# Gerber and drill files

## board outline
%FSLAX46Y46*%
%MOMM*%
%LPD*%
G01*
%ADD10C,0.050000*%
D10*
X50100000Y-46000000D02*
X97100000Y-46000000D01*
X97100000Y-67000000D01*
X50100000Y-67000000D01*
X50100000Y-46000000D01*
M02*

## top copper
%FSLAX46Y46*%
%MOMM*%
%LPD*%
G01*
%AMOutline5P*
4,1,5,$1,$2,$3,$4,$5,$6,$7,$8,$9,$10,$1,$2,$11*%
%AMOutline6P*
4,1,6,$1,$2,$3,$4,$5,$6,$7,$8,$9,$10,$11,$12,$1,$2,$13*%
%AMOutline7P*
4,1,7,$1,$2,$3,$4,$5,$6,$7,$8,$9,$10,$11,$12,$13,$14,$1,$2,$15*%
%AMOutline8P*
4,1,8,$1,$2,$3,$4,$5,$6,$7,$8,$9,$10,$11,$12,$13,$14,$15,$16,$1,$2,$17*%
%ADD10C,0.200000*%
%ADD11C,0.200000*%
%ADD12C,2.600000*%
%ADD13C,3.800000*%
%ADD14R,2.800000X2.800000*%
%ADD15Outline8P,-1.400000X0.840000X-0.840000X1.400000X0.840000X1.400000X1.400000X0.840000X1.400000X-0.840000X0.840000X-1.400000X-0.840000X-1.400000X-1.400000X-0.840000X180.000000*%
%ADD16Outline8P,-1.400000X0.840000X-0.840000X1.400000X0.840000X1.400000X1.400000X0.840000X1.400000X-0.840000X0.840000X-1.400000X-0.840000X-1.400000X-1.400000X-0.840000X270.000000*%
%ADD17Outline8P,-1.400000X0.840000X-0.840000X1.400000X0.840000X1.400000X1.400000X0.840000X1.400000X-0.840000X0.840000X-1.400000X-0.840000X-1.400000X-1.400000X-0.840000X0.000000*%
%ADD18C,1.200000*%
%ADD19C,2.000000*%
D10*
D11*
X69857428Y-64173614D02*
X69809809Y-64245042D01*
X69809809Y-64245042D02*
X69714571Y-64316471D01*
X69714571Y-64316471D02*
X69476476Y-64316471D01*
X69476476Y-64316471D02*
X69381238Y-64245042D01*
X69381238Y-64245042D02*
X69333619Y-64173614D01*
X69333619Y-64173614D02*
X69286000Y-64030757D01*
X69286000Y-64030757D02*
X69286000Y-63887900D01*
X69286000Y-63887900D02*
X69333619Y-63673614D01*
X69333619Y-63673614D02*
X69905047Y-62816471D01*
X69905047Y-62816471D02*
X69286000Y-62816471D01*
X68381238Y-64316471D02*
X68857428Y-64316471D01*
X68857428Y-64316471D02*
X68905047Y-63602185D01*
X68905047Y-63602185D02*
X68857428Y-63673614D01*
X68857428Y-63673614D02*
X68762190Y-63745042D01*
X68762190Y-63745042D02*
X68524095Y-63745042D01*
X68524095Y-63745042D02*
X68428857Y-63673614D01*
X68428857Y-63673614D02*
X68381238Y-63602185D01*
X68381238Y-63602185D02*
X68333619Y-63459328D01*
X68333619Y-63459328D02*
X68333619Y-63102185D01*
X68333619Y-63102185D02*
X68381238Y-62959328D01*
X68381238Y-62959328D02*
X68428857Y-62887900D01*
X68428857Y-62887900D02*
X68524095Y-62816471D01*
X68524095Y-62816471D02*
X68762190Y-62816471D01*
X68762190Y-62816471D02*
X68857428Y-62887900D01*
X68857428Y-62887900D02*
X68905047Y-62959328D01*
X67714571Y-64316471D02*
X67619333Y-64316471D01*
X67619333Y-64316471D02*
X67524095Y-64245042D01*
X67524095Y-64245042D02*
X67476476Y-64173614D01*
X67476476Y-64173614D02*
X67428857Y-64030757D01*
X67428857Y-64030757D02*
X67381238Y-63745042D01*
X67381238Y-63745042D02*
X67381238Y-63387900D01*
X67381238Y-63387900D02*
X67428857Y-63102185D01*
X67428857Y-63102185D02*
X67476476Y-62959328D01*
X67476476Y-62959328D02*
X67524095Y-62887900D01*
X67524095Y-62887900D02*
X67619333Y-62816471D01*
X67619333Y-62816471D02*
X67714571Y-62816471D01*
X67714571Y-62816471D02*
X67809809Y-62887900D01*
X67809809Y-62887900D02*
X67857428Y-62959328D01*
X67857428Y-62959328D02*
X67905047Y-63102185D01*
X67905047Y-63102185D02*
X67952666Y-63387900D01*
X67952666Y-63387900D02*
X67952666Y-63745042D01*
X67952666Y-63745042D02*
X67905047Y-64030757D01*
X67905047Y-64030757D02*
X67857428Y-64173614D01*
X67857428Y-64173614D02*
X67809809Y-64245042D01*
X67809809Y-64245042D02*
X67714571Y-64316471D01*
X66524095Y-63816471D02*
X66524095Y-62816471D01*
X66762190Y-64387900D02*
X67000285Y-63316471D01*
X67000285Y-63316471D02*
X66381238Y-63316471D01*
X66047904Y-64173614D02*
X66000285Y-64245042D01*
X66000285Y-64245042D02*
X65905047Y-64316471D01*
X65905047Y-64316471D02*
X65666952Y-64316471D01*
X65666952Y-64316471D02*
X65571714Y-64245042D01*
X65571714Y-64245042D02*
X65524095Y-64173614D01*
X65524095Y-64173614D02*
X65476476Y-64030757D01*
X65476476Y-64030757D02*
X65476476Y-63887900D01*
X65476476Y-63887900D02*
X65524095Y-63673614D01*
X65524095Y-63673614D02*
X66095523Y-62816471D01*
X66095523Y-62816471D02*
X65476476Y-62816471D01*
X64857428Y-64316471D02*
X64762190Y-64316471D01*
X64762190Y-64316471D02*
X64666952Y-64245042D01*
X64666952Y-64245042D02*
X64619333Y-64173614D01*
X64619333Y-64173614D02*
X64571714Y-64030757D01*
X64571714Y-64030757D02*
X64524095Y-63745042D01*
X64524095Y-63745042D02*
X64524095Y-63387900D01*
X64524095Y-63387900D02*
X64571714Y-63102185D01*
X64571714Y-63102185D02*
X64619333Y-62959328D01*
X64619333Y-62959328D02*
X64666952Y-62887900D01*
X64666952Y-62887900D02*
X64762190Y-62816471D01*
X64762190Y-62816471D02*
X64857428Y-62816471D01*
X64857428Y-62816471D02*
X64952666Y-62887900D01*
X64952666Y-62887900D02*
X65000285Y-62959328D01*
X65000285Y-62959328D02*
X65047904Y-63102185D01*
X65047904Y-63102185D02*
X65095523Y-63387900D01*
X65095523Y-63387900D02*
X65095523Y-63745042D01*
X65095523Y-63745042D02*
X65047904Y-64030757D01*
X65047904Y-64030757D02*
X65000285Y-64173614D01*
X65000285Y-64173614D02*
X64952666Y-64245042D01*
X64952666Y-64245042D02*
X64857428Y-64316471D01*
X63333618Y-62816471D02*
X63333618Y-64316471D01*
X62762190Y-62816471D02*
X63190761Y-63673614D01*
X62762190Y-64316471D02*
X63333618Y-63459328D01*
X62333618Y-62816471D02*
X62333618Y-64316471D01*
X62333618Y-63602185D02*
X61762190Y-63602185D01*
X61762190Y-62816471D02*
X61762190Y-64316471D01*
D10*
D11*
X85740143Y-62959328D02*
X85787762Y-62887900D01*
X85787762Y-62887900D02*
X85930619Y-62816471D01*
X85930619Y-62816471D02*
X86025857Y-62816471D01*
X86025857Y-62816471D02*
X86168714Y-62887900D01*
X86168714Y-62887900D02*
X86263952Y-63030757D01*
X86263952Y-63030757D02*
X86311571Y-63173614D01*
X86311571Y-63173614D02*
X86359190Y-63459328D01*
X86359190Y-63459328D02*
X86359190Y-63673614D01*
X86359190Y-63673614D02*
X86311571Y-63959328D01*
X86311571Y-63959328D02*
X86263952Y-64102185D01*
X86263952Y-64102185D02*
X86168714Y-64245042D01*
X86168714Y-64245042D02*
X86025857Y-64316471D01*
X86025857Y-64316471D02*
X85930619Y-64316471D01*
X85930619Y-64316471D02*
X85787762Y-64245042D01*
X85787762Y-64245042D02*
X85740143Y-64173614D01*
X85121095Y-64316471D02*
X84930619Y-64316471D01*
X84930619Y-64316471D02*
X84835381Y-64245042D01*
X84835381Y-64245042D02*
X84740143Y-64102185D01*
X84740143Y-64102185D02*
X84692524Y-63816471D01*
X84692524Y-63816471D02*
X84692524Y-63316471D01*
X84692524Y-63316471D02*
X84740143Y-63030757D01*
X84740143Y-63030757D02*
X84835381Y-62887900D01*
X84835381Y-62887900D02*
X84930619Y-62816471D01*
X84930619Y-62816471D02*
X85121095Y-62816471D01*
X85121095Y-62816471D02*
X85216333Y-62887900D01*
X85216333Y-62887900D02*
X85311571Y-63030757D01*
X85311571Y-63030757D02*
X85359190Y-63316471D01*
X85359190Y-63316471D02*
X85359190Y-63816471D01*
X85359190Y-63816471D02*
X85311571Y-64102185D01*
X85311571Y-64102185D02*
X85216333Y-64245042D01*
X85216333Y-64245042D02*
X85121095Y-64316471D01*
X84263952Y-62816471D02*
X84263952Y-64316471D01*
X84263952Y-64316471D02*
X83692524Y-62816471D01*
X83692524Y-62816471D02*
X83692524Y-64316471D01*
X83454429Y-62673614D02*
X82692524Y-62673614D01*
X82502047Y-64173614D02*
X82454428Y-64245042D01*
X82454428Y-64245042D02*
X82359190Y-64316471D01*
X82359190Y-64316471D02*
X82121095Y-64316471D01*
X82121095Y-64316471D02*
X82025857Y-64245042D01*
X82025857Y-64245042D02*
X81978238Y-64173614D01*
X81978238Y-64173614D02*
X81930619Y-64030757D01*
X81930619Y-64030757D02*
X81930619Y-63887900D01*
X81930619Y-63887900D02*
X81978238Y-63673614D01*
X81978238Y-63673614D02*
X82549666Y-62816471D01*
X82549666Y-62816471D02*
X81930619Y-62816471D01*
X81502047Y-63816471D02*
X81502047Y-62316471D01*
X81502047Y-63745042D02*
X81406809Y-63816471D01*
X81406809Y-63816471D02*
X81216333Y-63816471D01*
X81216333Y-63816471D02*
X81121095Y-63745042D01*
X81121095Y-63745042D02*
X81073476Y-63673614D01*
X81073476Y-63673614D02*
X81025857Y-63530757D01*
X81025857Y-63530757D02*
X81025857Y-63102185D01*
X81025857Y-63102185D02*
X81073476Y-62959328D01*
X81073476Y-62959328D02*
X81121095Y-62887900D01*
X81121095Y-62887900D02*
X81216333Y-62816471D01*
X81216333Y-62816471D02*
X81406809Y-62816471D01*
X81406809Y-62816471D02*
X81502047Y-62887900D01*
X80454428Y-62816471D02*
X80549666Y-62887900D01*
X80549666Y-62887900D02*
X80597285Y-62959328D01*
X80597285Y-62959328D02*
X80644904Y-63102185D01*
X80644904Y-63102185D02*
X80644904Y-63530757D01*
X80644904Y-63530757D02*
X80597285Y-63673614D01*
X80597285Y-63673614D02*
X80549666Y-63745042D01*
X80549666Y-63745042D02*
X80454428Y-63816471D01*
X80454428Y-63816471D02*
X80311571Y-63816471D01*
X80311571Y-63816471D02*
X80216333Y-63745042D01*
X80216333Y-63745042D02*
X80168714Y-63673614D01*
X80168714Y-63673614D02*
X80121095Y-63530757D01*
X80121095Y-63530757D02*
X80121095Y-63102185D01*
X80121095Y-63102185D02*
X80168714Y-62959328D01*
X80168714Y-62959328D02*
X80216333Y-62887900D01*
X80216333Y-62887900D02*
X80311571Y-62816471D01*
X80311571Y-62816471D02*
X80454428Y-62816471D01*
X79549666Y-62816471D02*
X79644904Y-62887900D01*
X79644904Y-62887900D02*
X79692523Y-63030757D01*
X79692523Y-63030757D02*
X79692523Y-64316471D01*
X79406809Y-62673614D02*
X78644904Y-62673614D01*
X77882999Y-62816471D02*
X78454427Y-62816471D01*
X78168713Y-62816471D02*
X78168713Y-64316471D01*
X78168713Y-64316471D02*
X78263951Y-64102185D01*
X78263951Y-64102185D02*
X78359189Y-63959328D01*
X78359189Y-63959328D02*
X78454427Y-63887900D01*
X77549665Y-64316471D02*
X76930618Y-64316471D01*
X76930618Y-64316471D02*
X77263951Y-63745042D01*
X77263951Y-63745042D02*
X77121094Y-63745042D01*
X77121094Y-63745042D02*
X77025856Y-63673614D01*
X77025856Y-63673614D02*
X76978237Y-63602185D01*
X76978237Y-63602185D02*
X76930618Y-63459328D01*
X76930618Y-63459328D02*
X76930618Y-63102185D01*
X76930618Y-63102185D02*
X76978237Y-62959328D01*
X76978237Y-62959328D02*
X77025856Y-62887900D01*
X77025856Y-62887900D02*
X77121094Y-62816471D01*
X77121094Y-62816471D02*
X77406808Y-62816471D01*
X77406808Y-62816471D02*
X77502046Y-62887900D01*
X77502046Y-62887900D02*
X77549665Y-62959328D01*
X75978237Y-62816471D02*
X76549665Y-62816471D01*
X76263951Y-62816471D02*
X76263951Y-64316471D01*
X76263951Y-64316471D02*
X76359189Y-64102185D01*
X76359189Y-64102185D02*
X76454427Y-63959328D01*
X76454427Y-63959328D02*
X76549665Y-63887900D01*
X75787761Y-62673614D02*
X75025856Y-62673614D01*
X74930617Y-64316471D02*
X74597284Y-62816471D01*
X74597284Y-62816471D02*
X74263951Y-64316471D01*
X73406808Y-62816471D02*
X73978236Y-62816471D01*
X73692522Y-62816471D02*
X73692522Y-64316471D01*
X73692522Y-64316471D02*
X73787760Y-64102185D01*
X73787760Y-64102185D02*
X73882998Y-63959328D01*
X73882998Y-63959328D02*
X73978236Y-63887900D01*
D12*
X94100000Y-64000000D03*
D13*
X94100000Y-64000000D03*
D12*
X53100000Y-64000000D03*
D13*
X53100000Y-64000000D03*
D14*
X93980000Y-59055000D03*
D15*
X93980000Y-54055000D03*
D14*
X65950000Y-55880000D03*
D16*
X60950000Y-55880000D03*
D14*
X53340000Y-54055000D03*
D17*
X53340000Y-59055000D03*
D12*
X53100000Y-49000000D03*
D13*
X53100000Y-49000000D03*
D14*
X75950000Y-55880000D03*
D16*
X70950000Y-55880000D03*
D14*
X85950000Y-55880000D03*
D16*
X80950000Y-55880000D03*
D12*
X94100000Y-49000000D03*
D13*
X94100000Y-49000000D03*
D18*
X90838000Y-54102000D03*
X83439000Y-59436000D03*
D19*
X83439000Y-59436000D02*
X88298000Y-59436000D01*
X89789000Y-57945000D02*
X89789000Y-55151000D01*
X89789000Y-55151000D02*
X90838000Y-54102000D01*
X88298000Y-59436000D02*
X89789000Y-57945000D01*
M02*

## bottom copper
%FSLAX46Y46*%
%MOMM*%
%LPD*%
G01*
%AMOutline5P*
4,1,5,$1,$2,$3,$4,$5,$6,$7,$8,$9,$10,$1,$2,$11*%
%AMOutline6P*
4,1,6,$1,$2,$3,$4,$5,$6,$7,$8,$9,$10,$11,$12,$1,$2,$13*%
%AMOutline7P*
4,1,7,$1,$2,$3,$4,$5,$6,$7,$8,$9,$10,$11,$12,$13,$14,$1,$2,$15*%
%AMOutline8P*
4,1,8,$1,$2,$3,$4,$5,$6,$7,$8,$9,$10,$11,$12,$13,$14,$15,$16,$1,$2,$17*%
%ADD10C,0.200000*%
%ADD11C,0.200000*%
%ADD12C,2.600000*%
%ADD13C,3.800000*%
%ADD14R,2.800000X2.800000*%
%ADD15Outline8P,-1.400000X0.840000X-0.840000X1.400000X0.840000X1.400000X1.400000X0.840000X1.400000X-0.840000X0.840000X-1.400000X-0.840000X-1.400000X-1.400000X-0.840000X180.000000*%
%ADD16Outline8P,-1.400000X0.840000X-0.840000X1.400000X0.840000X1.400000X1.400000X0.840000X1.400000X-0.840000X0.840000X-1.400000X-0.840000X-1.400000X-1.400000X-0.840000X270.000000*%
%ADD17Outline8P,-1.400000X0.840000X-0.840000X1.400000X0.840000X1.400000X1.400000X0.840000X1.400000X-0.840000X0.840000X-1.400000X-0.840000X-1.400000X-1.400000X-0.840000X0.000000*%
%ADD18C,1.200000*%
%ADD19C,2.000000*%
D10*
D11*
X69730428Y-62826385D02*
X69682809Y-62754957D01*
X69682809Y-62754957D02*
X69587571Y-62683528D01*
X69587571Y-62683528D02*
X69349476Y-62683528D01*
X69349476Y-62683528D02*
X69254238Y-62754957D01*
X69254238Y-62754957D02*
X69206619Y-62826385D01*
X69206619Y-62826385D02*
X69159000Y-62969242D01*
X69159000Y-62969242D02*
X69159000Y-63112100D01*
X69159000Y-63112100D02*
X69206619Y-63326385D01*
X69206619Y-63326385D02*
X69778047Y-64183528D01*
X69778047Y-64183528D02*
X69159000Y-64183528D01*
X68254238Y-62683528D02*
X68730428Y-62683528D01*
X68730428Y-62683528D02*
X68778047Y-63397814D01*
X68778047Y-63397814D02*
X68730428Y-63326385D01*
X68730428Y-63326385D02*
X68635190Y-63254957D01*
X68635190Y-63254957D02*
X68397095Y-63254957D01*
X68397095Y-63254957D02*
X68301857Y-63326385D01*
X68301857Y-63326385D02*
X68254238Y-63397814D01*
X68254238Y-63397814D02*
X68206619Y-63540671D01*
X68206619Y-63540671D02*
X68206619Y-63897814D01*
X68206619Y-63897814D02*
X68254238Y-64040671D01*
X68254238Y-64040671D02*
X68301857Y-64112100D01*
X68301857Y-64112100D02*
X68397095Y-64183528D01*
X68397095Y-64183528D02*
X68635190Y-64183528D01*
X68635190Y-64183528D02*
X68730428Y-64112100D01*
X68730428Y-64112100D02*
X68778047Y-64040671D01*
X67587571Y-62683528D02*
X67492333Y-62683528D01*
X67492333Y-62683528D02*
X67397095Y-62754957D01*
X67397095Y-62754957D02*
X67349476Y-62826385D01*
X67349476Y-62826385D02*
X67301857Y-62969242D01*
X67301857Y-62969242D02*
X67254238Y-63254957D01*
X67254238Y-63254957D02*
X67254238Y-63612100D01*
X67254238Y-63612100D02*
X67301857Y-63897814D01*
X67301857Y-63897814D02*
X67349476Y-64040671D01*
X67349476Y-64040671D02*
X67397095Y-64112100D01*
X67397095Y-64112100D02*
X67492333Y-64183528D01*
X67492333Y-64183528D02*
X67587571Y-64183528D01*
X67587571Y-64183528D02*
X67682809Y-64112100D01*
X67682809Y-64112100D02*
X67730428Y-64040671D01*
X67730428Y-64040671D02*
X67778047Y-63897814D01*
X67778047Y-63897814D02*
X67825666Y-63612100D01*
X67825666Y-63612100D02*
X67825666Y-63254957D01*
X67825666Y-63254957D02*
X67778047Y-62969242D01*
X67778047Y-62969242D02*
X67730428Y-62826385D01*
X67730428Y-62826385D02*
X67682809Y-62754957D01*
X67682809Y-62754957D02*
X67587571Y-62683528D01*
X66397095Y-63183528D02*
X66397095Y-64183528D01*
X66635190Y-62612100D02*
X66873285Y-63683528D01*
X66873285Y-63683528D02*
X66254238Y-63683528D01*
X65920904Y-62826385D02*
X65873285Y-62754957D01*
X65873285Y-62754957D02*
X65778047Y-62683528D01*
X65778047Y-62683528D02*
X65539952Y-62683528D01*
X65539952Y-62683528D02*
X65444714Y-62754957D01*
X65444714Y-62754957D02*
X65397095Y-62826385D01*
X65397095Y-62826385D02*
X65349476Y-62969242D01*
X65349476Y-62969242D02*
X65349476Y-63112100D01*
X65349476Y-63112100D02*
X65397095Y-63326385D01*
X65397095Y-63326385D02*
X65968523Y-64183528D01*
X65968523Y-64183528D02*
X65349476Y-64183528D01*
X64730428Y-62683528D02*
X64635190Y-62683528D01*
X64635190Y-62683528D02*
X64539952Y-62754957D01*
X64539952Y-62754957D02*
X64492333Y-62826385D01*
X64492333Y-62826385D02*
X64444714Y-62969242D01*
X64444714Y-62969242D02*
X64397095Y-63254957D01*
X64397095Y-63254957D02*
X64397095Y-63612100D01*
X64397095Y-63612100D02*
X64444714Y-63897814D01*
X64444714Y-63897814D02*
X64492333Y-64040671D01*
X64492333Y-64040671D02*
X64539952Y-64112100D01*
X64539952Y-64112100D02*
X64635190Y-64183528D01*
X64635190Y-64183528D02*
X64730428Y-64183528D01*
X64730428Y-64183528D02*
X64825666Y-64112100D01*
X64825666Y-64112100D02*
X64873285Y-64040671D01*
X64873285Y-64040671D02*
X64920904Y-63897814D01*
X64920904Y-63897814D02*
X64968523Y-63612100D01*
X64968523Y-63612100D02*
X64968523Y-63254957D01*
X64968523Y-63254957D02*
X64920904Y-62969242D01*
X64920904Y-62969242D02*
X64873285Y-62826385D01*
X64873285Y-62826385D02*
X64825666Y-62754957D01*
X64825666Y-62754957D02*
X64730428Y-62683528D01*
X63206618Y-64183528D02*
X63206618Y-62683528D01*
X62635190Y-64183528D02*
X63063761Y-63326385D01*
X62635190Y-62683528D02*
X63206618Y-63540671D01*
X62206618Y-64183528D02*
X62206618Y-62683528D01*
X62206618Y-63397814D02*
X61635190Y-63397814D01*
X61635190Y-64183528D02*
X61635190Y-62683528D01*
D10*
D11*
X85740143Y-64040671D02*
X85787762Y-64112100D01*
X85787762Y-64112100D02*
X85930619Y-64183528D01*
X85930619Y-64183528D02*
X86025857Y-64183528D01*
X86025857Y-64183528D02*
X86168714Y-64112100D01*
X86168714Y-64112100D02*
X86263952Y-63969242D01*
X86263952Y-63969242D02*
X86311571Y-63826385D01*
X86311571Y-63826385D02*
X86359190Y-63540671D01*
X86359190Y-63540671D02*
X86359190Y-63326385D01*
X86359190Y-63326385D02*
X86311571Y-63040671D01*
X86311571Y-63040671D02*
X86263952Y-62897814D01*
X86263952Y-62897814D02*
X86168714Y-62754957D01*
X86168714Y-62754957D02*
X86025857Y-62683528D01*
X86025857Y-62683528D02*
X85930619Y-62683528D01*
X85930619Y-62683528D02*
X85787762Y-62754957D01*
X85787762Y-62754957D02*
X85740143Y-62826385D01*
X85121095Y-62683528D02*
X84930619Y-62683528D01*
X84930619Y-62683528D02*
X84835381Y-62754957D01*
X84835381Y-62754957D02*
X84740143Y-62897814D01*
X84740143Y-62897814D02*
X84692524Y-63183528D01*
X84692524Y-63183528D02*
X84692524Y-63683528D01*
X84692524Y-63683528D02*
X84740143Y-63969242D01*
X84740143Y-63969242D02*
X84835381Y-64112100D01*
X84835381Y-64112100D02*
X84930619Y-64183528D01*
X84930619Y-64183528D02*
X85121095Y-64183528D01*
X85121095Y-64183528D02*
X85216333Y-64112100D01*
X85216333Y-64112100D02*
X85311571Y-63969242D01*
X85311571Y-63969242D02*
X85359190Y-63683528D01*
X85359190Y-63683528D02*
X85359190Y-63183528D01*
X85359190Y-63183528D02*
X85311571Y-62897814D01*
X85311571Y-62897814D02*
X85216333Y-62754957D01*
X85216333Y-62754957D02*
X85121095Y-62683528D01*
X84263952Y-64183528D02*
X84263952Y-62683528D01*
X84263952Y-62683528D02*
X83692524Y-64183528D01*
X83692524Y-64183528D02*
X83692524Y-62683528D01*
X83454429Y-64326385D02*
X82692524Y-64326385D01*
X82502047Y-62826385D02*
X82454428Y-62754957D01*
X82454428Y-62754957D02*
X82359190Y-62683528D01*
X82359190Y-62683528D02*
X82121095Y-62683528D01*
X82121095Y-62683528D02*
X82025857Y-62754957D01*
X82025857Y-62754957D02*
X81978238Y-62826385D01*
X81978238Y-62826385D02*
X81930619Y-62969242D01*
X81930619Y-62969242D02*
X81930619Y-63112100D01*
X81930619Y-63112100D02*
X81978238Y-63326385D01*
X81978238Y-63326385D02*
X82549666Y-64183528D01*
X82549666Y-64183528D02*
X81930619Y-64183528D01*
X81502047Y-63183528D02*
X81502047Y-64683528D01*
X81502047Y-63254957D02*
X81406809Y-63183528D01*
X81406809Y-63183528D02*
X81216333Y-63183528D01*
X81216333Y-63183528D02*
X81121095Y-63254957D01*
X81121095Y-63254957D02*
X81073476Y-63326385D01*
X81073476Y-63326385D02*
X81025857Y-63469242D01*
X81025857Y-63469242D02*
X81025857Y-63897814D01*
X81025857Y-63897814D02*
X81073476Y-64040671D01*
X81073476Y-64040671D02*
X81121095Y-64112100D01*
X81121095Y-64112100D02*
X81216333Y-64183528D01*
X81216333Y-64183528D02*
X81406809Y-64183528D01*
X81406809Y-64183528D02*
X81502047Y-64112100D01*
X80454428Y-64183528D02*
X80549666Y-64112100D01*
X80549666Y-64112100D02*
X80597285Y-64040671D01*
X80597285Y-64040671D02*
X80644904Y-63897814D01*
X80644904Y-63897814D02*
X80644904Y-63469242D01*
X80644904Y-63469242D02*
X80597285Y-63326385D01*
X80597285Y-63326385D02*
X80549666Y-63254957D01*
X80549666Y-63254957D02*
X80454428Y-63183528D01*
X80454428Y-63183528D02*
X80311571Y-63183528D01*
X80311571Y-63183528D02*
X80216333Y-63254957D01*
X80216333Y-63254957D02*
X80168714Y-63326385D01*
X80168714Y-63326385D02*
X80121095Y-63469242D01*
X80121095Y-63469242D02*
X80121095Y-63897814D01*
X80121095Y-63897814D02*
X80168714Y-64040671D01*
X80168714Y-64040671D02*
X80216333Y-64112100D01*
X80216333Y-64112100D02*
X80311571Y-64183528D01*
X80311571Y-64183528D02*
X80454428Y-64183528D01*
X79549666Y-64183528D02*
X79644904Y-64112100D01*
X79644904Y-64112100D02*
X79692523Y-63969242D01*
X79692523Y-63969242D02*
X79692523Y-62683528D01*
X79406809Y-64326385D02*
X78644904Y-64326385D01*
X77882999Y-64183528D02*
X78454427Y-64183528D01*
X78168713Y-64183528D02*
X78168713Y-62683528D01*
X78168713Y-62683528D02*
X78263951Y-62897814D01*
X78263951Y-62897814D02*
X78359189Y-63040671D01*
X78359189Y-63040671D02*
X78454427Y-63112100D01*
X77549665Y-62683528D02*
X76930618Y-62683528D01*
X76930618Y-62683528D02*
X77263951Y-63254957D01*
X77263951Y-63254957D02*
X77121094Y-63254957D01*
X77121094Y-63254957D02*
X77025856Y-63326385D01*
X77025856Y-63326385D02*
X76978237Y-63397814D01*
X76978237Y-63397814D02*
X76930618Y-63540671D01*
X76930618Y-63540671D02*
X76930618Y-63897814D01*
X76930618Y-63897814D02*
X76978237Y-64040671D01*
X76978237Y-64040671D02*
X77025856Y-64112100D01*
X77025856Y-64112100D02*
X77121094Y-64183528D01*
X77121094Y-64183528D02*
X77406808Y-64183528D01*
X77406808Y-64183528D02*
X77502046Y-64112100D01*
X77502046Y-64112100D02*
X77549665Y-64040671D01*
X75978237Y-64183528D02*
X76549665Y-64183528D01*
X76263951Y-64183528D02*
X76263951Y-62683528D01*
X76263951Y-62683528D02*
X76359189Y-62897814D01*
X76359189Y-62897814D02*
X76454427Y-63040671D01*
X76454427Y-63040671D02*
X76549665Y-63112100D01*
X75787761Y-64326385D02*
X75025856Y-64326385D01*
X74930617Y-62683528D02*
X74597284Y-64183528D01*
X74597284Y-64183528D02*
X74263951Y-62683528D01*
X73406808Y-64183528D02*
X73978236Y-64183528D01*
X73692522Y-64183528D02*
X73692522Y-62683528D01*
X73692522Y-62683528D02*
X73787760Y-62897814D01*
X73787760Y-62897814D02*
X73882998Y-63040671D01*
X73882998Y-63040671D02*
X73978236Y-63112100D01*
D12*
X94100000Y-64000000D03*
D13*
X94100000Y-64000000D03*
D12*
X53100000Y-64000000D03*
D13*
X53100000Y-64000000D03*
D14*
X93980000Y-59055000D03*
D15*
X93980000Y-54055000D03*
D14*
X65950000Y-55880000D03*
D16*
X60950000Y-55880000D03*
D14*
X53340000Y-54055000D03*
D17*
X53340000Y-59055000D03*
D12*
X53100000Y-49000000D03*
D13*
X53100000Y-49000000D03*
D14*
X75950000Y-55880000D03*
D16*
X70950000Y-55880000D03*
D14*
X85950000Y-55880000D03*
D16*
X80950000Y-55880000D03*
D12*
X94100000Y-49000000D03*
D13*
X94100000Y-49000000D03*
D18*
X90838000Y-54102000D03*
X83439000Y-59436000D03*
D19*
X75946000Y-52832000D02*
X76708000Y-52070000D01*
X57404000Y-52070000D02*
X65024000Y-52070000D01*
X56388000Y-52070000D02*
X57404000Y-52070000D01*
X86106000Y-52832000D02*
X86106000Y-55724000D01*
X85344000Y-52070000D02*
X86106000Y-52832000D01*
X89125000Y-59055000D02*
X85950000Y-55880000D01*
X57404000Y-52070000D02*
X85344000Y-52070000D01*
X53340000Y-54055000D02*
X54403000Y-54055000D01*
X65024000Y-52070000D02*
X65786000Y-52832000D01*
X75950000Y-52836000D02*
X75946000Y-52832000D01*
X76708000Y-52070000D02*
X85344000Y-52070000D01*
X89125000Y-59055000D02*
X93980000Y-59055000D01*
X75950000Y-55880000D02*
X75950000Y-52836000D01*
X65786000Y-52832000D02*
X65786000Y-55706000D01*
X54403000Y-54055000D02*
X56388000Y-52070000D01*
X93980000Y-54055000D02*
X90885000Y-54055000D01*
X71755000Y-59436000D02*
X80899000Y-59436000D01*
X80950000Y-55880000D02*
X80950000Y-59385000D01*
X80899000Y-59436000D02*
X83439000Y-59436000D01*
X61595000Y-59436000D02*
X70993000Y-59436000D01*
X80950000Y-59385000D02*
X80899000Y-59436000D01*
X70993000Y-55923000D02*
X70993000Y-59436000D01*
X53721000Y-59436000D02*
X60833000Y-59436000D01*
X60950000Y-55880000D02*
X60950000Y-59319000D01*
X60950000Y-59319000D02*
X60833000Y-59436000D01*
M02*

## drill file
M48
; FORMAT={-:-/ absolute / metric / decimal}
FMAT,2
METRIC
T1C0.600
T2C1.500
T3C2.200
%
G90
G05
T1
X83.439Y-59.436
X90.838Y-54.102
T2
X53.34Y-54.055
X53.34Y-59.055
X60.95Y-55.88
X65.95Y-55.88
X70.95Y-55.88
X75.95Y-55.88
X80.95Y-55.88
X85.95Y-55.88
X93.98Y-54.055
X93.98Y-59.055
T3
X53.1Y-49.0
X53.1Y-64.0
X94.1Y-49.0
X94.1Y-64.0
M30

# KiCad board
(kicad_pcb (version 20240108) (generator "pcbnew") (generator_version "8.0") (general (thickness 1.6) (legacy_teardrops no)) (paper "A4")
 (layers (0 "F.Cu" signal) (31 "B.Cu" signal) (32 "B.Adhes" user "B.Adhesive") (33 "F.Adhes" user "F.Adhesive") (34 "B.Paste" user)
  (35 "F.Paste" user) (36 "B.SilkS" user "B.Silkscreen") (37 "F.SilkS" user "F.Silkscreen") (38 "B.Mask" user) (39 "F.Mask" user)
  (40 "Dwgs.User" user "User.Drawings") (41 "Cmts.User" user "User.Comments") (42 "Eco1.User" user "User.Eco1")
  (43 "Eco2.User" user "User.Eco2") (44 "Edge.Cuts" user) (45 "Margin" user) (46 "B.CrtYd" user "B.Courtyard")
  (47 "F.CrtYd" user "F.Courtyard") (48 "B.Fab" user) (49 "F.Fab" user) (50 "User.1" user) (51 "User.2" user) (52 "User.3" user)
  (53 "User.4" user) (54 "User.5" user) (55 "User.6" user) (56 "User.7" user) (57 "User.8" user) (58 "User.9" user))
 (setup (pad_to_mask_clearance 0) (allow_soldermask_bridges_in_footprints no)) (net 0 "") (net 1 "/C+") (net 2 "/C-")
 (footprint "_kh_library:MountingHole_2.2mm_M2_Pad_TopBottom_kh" (layer "F.Cu") (at 94.1 64)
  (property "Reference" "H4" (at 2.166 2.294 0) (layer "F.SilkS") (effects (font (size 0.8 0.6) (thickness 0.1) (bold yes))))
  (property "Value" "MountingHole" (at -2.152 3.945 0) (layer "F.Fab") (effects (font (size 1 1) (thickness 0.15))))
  (pad "1" thru_hole circle (at 0 0) (size 2.6 2.6) (drill 2.2) (layers "*.Cu" "*.Mask") (remove_unused_layers no))
  (pad "1" connect circle (at 0 0) (size 3.8 3.8) (layers "F.Cu" "F.Mask"))
  (pad "1" connect circle (at 0 0) (size 3.8 3.8) (layers "B.Cu" "B.Mask")))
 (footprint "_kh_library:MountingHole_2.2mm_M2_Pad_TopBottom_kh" (layer "F.Cu") (at 53.1 64)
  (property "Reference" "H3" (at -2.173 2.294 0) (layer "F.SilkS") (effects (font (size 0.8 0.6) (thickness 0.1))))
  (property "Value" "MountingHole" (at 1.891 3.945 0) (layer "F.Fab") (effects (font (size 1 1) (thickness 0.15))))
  (pad "1" thru_hole circle (at 0 0) (size 2.6 2.6) (drill 2.2) (layers "*.Cu" "*.Mask") (remove_unused_layers no))
  (pad "1" connect circle (at 0 0) (size 3.8 3.8) (layers "F.Cu" "F.Mask"))
  (pad "1" connect circle (at 0 0) (size 3.8 3.8) (layers "B.Cu" "B.Mask")))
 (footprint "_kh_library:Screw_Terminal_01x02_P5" (layer "F.Cu") (at 93.98 59.055 180)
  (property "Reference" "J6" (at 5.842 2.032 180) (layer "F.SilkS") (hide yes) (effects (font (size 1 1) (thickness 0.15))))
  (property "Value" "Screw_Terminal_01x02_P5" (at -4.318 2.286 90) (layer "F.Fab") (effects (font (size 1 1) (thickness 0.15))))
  (pad "1" thru_hole rect (at 0 0 180) (size 2.8 2.8) (drill 1.5) (layers "*.Cu" "*.Mask") (remove_unused_layers no) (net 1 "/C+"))
  (pad "2" thru_hole roundrect (at 0 5 180) (size 2.8 2.8) (drill 1.5) (layers "*.Cu" "*.Mask") (remove_unused_layers no)
   (roundrect_rratio 0) (chamfer_ratio 0.2) (chamfer top_left top_right bottom_left bottom_right) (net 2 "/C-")))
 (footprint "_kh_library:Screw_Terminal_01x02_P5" (layer "F.Cu") (at 65.95 55.88 -90)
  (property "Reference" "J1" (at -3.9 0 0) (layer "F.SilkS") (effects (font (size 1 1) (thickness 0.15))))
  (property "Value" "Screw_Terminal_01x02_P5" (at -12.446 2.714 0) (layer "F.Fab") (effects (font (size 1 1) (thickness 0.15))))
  (pad "1" thru_hole rect (at 0 0 270) (size 2.8 2.8) (drill 1.5) (layers "*.Cu" "*.Mask") (remove_unused_layers no) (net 1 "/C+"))
  (pad "2" thru_hole roundrect (at 0 5 270) (size 2.8 2.8) (drill 1.5) (layers "*.Cu" "*.Mask") (remove_unused_layers no)
   (roundrect_rratio 0) (chamfer_ratio 0.2) (chamfer top_left top_right bottom_left bottom_right) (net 2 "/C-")))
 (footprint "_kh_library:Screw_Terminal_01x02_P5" (layer "F.Cu") (at 53.34 54.055)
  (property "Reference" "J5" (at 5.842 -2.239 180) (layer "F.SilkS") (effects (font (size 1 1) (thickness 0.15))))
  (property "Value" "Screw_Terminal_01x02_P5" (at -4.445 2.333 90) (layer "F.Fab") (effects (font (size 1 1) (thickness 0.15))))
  (pad "1" thru_hole rect (at 0 0) (size 2.8 2.8) (drill 1.5) (layers "*.Cu" "*.Mask") (remove_unused_layers no) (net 1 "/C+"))
  (pad "2" thru_hole roundrect (at 0 5) (size 2.8 2.8) (drill 1.5) (layers "*.Cu" "*.Mask") (remove_unused_layers no) (roundrect_rratio 0)
   (chamfer_ratio 0.2) (chamfer top_left top_right bottom_left bottom_right) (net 2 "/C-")))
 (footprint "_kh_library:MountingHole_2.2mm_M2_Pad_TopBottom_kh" (layer "F.Cu") (at 53.1 49)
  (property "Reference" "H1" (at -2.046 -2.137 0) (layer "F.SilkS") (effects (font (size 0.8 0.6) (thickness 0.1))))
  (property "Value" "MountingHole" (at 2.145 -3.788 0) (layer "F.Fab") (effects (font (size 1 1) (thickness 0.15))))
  (pad "1" thru_hole circle (at 0 0) (size 2.6 2.6) (drill 2.2) (layers "*.Cu" "*.Mask") (remove_unused_layers no))
  (pad "1" connect circle (at 0 0) (size 3.8 3.8) (layers "F.Cu" "F.Mask"))
  (pad "1" connect circle (at 0 0) (size 3.8 3.8) (layers "B.Cu" "B.Mask")))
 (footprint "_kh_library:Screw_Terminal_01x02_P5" (layer "F.Cu") (at 75.95 55.88 -90)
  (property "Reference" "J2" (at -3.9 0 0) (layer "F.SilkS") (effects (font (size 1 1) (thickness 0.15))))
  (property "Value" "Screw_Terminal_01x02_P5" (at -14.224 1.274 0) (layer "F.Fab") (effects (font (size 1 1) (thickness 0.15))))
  (pad "1" thru_hole rect (at 0 0 270) (size 2.8 2.8) (drill 1.5) (layers "*.Cu" "*.Mask") (remove_unused_layers no) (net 1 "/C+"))
  (pad "2" thru_hole roundrect (at 0 5 270) (size 2.8 2.8) (drill 1.5) (layers "*.Cu" "*.Mask") (remove_unused_layers no)
   (roundrect_rratio 0) (chamfer_ratio 0.2) (chamfer top_left top_right bottom_left bottom_right) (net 2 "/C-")))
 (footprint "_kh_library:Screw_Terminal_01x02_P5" (layer "F.Cu") (at 85.95 55.88 -90)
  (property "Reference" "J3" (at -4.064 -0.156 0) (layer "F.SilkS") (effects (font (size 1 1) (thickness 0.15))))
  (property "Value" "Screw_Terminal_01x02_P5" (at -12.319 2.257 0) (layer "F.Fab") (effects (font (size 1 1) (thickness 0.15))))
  (pad "1" thru_hole rect (at 0 0 270) (size 2.8 2.8) (drill 1.5) (layers "*.Cu" "*.Mask") (remove_unused_layers no) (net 1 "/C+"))
  (pad "2" thru_hole roundrect (at 0 5 270) (size 2.8 2.8) (drill 1.5) (layers "*.Cu" "*.Mask") (remove_unused_layers no)
   (roundrect_rratio 0) (chamfer_ratio 0.2) (chamfer top_left top_right bottom_left bottom_right) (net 2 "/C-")))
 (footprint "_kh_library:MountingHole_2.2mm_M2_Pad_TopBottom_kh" (layer "F.Cu") (at 94.1 49)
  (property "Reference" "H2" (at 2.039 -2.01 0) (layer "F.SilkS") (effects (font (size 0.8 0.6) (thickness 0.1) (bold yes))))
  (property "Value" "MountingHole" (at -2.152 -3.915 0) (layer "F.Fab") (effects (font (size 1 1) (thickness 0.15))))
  (pad "1" thru_hole circle (at 0 0) (size 2.6 2.6) (drill 2.2) (layers "*.Cu" "*.Mask") (remove_unused_layers no))
  (pad "1" connect circle (at 0 0) (size 3.8 3.8) (layers "F.Cu" "F.Mask"))
  (pad "1" connect circle (at 0 0) (size 3.8 3.8) (layers "B.Cu" "B.Mask")))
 (gr_rect (start 50.1 46) (end 97.1 67) (stroke (width 0.05) (type default)) (fill none) (layer "Edge.Cuts"))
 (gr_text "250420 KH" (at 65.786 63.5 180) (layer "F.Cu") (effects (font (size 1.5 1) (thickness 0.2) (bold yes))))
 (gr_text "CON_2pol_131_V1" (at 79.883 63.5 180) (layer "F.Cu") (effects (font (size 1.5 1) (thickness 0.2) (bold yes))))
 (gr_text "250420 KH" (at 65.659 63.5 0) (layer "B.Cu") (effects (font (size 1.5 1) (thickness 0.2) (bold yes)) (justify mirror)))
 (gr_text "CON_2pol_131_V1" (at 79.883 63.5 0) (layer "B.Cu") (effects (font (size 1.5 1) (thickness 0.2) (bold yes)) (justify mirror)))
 (segment (start 75.946 52.832) (end 76.708 52.07) (width 2) (layer "B.Cu") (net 1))
 (segment (start 57.404 52.07) (end 65.024 52.07) (width 2) (layer "B.Cu") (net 1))
 (segment (start 56.388 52.07) (end 57.404 52.07) (width 2) (layer "B.Cu") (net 1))
 (segment (start 86.106 52.832) (end 86.106 55.724) (width 2) (layer "B.Cu") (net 1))
 (segment (start 85.344 52.07) (end 86.106 52.832) (width 2) (layer "B.Cu") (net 1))
 (segment (start 89.125 59.055) (end 85.95 55.88) (width 2) (layer "B.Cu") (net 1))
 (segment (start 57.404 52.07) (end 85.344 52.07) (width 2) (layer "B.Cu") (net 1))
 (segment (start 53.34 54.055) (end 54.403 54.055) (width 2) (layer "B.Cu") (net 1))
 (segment (start 65.024 52.07) (end 65.786 52.832) (width 2) (layer "B.Cu") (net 1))
 (segment (start 75.95 52.836) (end 75.946 52.832) (width 2) (layer "B.Cu") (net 1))
 (segment (start 76.708 52.07) (end 85.344 52.07) (width 2) (layer "B.Cu") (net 1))
 (segment (start 89.125 59.055) (end 93.98 59.055) (width 2) (layer "B.Cu") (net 1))
 (segment (start 75.95 55.88) (end 75.95 52.836) (width 2) (layer "B.Cu") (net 1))
 (segment (start 65.786 52.832) (end 65.786 55.706) (width 2) (layer "B.Cu") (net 1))
 (segment (start 54.403 54.055) (end 56.388 52.07) (width 2) (layer "B.Cu") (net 1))
 (segment (start 83.439 59.436) (end 88.298 59.436) (width 2) (layer "F.Cu") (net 2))
 (segment (start 89.789 57.945) (end 89.789 55.151) (width 2) (layer "F.Cu") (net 2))
 (segment (start 89.789 55.151) (end 90.838 54.102) (width 2) (layer "F.Cu") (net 2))
 (segment (start 88.298 59.436) (end 89.789 57.945) (width 2) (layer "F.Cu") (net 2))
 (via (at 90.838 54.102) (size 1.2) (drill 0.6) (layers "F.Cu" "B.Cu") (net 2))
 (via (at 83.439 59.436) (size 1.2) (drill 0.6) (layers "F.Cu" "B.Cu") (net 2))
 (segment (start 93.98 54.055) (end 90.885 54.055) (width 2) (layer "B.Cu") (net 2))
 (segment (start 71.755 59.436) (end 80.899 59.436) (width 2) (layer "B.Cu") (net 2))
 (segment (start 80.95 55.88) (end 80.95 59.385) (width 2) (layer "B.Cu") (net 2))
 (segment (start 80.899 59.436) (end 83.439 59.436) (width 2) (layer "B.Cu") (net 2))
 (segment (start 61.595 59.436) (end 70.993 59.436) (width 2) (layer "B.Cu") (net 2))
 (segment (start 80.95 59.385) (end 80.899 59.436) (width 2) (layer "B.Cu") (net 2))
 (segment (start 70.993 55.923) (end 70.993 59.436) (width 2) (layer "B.Cu") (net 2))
 (segment (start 53.721 59.436) (end 60.833 59.436) (width 2) (layer "B.Cu") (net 2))
 (segment (start 60.95 55.88) (end 60.95 59.319) (width 2) (layer "B.Cu") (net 2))
 (segment (start 60.95 59.319) (end 60.833 59.436) (width 2) (layer "B.Cu") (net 2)))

